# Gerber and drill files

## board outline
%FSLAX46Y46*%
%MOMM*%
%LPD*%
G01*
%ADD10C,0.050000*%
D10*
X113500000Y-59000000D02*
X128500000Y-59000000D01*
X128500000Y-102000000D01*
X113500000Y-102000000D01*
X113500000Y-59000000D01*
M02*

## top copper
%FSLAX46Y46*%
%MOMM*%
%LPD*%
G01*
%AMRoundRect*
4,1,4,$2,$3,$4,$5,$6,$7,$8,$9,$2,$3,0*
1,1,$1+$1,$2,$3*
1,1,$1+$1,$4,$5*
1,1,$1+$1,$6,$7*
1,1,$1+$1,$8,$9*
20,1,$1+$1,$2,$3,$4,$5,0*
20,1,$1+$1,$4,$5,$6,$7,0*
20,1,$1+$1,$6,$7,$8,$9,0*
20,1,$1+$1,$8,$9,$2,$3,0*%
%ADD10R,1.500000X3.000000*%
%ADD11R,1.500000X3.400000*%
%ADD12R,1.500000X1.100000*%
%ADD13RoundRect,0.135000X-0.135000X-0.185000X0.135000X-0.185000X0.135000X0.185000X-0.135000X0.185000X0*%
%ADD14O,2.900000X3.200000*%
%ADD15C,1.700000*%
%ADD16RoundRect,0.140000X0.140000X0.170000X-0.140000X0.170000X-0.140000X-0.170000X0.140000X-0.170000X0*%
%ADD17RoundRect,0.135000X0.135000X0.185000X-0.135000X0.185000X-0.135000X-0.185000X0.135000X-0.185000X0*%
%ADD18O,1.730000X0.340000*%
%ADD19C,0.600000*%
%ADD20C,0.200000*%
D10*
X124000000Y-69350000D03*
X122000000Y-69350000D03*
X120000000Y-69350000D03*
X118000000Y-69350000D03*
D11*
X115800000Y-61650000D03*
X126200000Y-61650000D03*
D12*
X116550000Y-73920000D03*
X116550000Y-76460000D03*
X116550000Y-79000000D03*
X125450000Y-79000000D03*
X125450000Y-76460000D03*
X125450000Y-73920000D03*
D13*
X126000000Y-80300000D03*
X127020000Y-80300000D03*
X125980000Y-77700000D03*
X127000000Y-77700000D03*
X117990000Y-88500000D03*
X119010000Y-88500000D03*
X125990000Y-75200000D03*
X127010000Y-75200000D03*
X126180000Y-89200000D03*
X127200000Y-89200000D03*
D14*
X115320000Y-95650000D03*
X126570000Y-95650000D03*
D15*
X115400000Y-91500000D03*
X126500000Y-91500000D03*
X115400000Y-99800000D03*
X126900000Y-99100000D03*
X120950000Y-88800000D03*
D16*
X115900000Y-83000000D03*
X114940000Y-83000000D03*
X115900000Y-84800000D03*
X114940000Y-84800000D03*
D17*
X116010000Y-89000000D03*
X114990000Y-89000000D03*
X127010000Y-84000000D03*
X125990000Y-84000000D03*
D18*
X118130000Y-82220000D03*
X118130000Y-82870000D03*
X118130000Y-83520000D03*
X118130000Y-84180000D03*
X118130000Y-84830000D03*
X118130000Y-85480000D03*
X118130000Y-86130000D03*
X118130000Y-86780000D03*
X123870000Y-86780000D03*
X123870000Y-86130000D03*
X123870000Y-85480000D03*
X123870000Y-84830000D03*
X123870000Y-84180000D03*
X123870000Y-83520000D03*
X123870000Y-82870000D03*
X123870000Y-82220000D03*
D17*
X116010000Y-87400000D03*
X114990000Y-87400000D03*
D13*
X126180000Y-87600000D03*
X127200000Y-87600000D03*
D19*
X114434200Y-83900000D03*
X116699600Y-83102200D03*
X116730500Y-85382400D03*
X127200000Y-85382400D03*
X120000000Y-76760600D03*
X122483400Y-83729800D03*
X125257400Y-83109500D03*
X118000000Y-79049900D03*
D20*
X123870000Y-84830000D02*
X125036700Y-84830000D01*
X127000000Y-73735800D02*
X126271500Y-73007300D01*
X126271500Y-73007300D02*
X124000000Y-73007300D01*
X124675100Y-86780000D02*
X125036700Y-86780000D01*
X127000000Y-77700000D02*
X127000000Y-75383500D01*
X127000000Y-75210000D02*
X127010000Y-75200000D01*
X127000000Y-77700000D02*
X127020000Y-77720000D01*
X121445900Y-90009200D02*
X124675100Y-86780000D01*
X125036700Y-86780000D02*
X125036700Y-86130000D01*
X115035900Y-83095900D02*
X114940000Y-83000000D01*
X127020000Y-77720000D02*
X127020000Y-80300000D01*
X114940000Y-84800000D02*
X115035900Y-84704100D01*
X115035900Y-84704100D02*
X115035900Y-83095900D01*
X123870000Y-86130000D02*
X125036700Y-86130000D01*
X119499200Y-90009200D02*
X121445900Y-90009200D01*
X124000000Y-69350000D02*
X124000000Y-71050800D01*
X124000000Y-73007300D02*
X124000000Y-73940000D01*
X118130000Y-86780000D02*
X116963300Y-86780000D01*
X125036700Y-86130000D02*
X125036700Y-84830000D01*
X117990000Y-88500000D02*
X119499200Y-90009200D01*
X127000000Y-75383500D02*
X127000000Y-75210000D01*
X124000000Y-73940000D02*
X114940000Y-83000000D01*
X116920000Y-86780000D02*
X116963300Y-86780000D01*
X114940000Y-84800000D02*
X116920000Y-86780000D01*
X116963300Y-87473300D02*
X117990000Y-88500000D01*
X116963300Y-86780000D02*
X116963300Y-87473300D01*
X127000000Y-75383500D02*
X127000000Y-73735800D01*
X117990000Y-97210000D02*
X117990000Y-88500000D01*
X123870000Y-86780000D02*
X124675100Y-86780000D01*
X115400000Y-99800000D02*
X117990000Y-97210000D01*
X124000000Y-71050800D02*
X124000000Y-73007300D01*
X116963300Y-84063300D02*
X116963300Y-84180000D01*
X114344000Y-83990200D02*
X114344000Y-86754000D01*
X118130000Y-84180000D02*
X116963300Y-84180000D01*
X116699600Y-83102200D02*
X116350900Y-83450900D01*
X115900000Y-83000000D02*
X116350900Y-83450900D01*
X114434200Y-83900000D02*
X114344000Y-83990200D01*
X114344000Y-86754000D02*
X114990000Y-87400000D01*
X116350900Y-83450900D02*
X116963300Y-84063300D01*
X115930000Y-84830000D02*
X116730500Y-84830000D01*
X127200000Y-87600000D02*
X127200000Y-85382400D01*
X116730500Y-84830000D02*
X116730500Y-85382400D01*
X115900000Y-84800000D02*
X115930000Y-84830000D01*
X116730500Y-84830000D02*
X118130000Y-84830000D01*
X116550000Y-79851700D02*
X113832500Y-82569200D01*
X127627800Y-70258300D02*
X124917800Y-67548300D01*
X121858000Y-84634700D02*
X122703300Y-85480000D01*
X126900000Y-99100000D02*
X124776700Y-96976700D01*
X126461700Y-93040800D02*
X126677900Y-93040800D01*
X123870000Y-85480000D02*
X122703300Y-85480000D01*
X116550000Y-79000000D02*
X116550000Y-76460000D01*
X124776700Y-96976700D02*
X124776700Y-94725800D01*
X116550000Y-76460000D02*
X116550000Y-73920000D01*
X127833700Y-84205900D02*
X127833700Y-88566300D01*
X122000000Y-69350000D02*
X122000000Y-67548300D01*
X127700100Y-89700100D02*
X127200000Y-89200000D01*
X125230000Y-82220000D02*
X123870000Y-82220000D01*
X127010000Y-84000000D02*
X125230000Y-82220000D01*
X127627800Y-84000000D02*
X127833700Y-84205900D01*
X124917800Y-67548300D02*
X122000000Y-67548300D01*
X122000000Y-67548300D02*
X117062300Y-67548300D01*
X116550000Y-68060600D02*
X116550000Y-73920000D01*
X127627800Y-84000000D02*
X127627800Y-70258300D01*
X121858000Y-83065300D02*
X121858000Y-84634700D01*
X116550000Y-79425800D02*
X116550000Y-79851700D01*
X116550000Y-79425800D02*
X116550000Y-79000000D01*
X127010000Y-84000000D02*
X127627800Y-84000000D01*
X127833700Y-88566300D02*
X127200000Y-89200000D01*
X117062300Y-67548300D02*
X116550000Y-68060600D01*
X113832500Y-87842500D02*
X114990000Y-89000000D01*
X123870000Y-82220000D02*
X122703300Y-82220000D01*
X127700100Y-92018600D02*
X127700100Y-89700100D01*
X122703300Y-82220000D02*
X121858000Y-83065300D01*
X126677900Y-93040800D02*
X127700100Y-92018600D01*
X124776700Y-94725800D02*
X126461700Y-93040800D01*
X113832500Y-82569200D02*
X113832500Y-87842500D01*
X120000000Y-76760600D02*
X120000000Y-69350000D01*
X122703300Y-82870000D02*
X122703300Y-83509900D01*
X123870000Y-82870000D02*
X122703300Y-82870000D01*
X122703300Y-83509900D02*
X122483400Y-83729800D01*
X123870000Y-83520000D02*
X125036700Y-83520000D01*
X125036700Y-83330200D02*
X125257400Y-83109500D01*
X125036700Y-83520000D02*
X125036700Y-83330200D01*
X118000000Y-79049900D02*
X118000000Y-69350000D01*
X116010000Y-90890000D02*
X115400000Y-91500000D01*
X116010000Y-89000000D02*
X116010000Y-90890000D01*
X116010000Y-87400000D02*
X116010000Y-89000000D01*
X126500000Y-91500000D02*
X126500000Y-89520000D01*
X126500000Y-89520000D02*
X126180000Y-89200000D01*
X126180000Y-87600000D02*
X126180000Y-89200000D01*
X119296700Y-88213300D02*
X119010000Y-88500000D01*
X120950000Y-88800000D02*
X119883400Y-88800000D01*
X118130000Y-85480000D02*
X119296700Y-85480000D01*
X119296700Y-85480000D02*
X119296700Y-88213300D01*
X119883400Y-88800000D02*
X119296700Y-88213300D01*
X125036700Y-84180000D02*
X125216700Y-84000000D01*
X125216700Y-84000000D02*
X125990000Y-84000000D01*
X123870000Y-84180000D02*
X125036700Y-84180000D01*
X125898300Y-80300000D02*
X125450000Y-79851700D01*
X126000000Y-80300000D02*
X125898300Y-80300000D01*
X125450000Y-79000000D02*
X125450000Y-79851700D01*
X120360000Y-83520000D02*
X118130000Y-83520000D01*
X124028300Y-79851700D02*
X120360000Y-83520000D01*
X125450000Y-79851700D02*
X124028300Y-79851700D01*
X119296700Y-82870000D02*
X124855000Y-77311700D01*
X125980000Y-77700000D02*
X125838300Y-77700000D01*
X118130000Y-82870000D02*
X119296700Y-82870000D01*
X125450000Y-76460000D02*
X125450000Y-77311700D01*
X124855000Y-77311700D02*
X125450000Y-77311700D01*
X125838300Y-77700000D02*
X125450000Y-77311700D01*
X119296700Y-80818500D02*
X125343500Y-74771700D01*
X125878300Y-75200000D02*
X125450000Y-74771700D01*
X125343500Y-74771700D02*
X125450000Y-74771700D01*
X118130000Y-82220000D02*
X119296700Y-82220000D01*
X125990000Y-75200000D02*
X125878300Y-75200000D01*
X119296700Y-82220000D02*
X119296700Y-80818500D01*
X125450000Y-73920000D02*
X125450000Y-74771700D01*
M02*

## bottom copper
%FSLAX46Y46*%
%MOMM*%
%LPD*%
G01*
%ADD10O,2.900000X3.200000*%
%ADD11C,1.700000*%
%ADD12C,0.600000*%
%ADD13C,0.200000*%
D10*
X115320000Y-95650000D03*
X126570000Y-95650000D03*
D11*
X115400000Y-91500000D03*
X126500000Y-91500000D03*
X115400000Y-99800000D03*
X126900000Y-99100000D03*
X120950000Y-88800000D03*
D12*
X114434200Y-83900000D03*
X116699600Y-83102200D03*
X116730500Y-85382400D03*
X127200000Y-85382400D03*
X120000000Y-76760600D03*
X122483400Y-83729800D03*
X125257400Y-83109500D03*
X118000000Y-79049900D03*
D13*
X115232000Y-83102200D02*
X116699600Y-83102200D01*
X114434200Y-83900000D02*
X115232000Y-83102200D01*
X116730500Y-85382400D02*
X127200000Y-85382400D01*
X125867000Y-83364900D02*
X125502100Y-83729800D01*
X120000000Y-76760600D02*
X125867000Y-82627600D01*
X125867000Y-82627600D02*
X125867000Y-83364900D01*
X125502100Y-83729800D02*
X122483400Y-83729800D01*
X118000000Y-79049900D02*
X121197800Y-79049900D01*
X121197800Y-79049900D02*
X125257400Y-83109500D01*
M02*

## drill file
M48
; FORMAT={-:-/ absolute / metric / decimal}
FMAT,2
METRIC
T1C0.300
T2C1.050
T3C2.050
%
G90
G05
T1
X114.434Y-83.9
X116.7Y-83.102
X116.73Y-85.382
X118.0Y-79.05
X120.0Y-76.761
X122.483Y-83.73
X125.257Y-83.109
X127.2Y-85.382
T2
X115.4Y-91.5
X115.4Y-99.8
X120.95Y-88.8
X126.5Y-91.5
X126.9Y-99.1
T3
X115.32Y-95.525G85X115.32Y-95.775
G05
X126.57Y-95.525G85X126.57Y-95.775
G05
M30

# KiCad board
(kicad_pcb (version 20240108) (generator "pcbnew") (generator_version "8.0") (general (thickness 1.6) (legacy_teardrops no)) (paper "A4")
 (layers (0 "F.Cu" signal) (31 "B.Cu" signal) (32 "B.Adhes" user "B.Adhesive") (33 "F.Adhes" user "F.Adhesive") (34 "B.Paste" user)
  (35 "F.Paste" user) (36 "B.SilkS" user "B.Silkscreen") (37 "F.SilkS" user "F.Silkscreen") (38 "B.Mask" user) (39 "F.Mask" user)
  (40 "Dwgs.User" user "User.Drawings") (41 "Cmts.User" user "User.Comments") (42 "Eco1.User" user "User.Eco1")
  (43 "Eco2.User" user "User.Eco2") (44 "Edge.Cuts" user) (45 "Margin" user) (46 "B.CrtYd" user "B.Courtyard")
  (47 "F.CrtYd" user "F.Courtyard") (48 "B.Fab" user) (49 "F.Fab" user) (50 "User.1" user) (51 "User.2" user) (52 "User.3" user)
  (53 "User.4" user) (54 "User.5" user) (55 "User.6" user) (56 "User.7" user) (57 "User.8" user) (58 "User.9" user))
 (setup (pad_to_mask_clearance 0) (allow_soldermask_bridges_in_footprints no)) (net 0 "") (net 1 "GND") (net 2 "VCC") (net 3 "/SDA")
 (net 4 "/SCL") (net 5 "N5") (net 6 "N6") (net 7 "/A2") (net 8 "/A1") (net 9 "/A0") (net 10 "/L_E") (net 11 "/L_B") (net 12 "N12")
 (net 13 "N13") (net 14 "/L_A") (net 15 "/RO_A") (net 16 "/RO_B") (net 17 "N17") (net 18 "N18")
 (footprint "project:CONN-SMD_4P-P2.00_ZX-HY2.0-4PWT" (layer "F.Cu") (at 121 65.5 180)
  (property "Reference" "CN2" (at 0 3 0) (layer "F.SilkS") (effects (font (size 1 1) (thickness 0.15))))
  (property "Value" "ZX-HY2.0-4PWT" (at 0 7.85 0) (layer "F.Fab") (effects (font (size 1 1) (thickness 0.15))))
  (pad "1" smd rect (at -3 -3.85 180) (size 1.5 3) (layers "F.Cu" "F.Paste" "F.Mask") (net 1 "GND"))
  (pad "2" smd rect (at -1 -3.85 180) (size 1.5 3) (layers "F.Cu" "F.Paste" "F.Mask") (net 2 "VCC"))
  (pad "3" smd rect (at 1 -3.85 180) (size 1.5 3) (layers "F.Cu" "F.Paste" "F.Mask") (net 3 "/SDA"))
  (pad "4" smd rect (at 3 -3.85 180) (size 1.5 3) (layers "F.Cu" "F.Paste" "F.Mask") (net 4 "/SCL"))
  (pad "5" smd rect (at 5.2 3.85 180) (size 1.5 3.4) (layers "F.Cu" "F.Paste" "F.Mask") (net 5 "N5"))
  (pad "6" smd rect (at -5.2 3.85 180) (size 1.5 3.4) (layers "F.Cu" "F.Paste" "F.Mask") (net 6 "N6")))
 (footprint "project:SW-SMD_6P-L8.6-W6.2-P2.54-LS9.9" (layer "F.Cu") (at 121 76.46 -90)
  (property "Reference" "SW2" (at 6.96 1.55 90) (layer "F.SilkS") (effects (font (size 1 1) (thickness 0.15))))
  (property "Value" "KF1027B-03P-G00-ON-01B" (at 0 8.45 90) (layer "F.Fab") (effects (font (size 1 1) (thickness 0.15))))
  (pad "1" smd rect (at -2.54 4.45 180) (size 1.5 1.1) (layers "F.Cu" "F.Paste" "F.Mask") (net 2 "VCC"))
  (pad "2" smd rect (at 0 4.45 180) (size 1.5 1.1) (layers "F.Cu" "F.Paste" "F.Mask") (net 2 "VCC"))
  (pad "3" smd rect (at 2.54 4.45 180) (size 1.5 1.1) (layers "F.Cu" "F.Paste" "F.Mask") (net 2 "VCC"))
  (pad "4" smd rect (at 2.54 -4.45 180) (size 1.5 1.1) (layers "F.Cu" "F.Paste" "F.Mask") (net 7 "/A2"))
  (pad "5" smd rect (at 0 -4.45 180) (size 1.5 1.1) (layers "F.Cu" "F.Paste" "F.Mask") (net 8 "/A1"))
  (pad "6" smd rect (at -2.54 -4.45 180) (size 1.5 1.1) (layers "F.Cu" "F.Paste" "F.Mask") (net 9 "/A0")))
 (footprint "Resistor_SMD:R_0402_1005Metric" (layer "F.Cu") (at 126.51 80.3)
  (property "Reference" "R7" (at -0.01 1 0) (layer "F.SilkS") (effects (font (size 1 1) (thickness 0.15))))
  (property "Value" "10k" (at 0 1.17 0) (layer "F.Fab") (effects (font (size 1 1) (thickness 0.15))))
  (pad "1" smd roundrect (at -0.51 0) (size 0.54 0.64) (layers "F.Cu" "F.Paste" "F.Mask") (roundrect_rratio 0.25) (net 7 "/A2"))
  (pad "2" smd roundrect (at 0.51 0) (size 0.54 0.64) (layers "F.Cu" "F.Paste" "F.Mask") (roundrect_rratio 0.25) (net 1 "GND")))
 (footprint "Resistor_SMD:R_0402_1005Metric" (layer "F.Cu") (at 126.49 77.7)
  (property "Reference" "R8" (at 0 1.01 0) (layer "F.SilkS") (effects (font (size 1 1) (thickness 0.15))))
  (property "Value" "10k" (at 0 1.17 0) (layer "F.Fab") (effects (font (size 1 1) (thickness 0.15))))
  (pad "1" smd roundrect (at -0.51 0) (size 0.54 0.64) (layers "F.Cu" "F.Paste" "F.Mask") (roundrect_rratio 0.25) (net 8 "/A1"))
  (pad "2" smd roundrect (at 0.51 0) (size 0.54 0.64) (layers "F.Cu" "F.Paste" "F.Mask") (roundrect_rratio 0.25) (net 1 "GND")))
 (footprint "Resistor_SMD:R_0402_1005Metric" (layer "F.Cu") (at 118.5 88.5)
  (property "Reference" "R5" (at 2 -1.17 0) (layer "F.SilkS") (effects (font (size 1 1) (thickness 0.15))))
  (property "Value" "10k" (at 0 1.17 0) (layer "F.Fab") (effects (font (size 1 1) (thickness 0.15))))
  (pad "1" smd roundrect (at -0.51 0) (size 0.54 0.64) (layers "F.Cu" "F.Paste" "F.Mask") (roundrect_rratio 0.25) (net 1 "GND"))
  (pad "2" smd roundrect (at 0.51 0) (size 0.54 0.64) (layers "F.Cu" "F.Paste" "F.Mask") (roundrect_rratio 0.25) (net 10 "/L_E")))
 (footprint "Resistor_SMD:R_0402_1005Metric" (layer "F.Cu") (at 126.5 75.2)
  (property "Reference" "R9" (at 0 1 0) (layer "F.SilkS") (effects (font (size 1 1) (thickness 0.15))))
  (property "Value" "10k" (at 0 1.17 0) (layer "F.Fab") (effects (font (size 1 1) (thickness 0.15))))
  (pad "1" smd roundrect (at -0.51 0) (size 0.54 0.64) (layers "F.Cu" "F.Paste" "F.Mask") (roundrect_rratio 0.25) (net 9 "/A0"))
  (pad "2" smd roundrect (at 0.51 0) (size 0.54 0.64) (layers "F.Cu" "F.Paste" "F.Mask") (roundrect_rratio 0.25) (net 1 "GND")))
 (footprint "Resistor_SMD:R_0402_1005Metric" (layer "F.Cu") (at 126.69 89.2)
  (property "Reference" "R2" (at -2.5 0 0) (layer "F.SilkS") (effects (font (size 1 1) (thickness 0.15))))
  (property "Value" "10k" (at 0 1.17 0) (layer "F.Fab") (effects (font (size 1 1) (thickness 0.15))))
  (pad "1" smd roundrect (at -0.51 0) (size 0.54 0.64) (layers "F.Cu" "F.Paste" "F.Mask") (roundrect_rratio 0.25) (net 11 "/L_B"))
  (pad "2" smd roundrect (at 0.51 0) (size 0.54 0.64) (layers "F.Cu" "F.Paste" "F.Mask") (roundrect_rratio 0.25) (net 2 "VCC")))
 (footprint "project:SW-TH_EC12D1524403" (layer "F.Cu") (at 121.11 94.3)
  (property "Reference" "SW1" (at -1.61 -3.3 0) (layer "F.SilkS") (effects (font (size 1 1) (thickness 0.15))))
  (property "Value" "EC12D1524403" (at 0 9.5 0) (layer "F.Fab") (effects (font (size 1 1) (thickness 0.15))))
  (pad "6" thru_hole oval (at -5.79 1.35) (size 2.9 3.2) (drill oval 2.049983 2.299995) (layers "*.Cu" "*.Mask") (remove_unused_layers no)
   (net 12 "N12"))
  (pad "7" thru_hole oval (at 5.46 1.35) (size 2.9 3.2) (drill oval 2.049983 2.299995) (layers "*.Cu" "*.Mask") (remove_unused_layers no)
   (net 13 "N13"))
  (pad "A" thru_hole circle (at -5.71 -2.8) (size 1.7 1.7) (drill 1.049985) (layers "*.Cu" "*.Mask") (remove_unused_layers no)
   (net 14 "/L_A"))
  (pad "B" thru_hole circle (at 5.39 -2.8) (size 1.7 1.7) (drill 1.049985) (layers "*.Cu" "*.Mask") (remove_unused_layers no)
   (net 11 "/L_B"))
  (pad "C" thru_hole circle (at -5.71 5.5) (size 1.7 1.7) (drill 1.049985) (layers "*.Cu" "*.Mask") (remove_unused_layers no) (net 1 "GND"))
  (pad "D" thru_hole circle (at 5.79 4.8) (size 1.7 1.7) (drill 1.049985) (layers "*.Cu" "*.Mask") (remove_unused_layers no) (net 2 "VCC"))
  (pad "E" thru_hole circle (at -0.16 -5.5) (size 1.7 1.7) (drill 1.049985) (layers "*.Cu" "*.Mask") (remove_unused_layers no)
   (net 10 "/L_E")))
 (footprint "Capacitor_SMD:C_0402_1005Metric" (layer "F.Cu") (at 115.42 83 180)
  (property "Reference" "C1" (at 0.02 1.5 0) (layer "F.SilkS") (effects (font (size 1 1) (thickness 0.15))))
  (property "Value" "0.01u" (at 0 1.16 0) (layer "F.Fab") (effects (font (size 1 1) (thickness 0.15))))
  (pad "1" smd roundrect (at -0.48 0 180) (size 0.56 0.62) (layers "F.Cu" "F.Paste" "F.Mask") (roundrect_rratio 0.25) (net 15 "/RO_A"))
  (pad "2" smd roundrect (at 0.48 0 180) (size 0.56 0.62) (layers "F.Cu" "F.Paste" "F.Mask") (roundrect_rratio 0.25) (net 1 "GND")))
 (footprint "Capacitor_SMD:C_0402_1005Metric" (layer "F.Cu") (at 115.42 84.8 180)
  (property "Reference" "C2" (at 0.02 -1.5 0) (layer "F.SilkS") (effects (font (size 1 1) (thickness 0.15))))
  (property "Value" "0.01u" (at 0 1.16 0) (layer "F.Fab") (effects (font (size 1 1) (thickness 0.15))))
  (pad "1" smd roundrect (at -0.48 0 180) (size 0.56 0.62) (layers "F.Cu" "F.Paste" "F.Mask") (roundrect_rratio 0.25) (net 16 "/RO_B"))
  (pad "2" smd roundrect (at 0.48 0 180) (size 0.56 0.62) (layers "F.Cu" "F.Paste" "F.Mask") (roundrect_rratio 0.25) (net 1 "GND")))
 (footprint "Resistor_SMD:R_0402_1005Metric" (layer "F.Cu") (at 115.5 89 180)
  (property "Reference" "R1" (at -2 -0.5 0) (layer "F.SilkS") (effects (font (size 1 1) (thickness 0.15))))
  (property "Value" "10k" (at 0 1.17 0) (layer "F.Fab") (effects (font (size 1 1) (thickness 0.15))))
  (pad "1" smd roundrect (at -0.51 0 180) (size 0.54 0.64) (layers "F.Cu" "F.Paste" "F.Mask") (roundrect_rratio 0.25) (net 14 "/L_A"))
  (pad "2" smd roundrect (at 0.51 0 180) (size 0.54 0.64) (layers "F.Cu" "F.Paste" "F.Mask") (roundrect_rratio 0.25) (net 2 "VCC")))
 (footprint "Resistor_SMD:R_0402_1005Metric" (layer "F.Cu") (at 126.5 84 180)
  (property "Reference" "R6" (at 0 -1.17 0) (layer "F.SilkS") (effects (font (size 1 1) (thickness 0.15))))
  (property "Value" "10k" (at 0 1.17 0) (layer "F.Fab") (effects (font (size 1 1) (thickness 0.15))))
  (pad "1" smd roundrect (at -0.51 0 180) (size 0.54 0.64) (layers "F.Cu" "F.Paste" "F.Mask") (roundrect_rratio 0.25) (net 2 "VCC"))
  (pad "2" smd roundrect (at 0.51 0 180) (size 0.54 0.64) (layers "F.Cu" "F.Paste" "F.Mask") (roundrect_rratio 0.25) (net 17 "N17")))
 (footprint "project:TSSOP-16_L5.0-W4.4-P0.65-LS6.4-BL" (layer "F.Cu") (at 121 84.5 -90)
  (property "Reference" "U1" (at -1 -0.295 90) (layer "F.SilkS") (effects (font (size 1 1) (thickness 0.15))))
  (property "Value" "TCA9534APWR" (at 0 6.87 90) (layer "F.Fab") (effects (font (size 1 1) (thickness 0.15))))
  (pad "1" smd oval (at -2.28 2.87 270) (size 0.34 1.73) (layers "F.Cu" "F.Paste" "F.Mask") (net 9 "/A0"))
  (pad "2" smd oval (at -1.63 2.87 270) (size 0.34 1.73) (layers "F.Cu" "F.Paste" "F.Mask") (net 8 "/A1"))
  (pad "3" smd oval (at -0.98 2.87 270) (size 0.34 1.73) (layers "F.Cu" "F.Paste" "F.Mask") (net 7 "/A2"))
  (pad "4" smd oval (at -0.32 2.87 270) (size 0.34 1.73) (layers "F.Cu" "F.Paste" "F.Mask") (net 15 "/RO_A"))
  (pad "5" smd oval (at 0.33 2.87 270) (size 0.34 1.73) (layers "F.Cu" "F.Paste" "F.Mask") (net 16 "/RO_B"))
  (pad "6" smd oval (at 0.98 2.87 270) (size 0.34 1.73) (layers "F.Cu" "F.Paste" "F.Mask") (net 10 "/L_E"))
  (pad "7" smd oval (at 1.63 2.87 270) (size 0.34 1.73) (layers "F.Cu" "F.Paste" "F.Mask") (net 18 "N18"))
  (pad "8" smd oval (at 2.28 2.87 270) (size 0.34 1.73) (layers "F.Cu" "F.Paste" "F.Mask") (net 1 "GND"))
  (pad "9" smd oval (at 2.28 -2.87 270) (size 0.34 1.73) (layers "F.Cu" "F.Paste" "F.Mask") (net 1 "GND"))
  (pad "10" smd oval (at 1.63 -2.87 270) (size 0.34 1.73) (layers "F.Cu" "F.Paste" "F.Mask") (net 1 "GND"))
  (pad "11" smd oval (at 0.98 -2.87 270) (size 0.34 1.73) (layers "F.Cu" "F.Paste" "F.Mask") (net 2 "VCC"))
  (pad "12" smd oval (at 0.33 -2.87 270) (size 0.34 1.73) (layers "F.Cu" "F.Paste" "F.Mask") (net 1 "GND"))
  (pad "13" smd oval (at -0.32 -2.87 270) (size 0.34 1.73) (layers "F.Cu" "F.Paste" "F.Mask") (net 17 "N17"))
  (pad "14" smd oval (at -0.98 -2.87 270) (size 0.34 1.73) (layers "F.Cu" "F.Paste" "F.Mask") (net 4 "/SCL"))
  (pad "15" smd oval (at -1.63 -2.87 270) (size 0.34 1.73) (layers "F.Cu" "F.Paste" "F.Mask") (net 3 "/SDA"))
  (pad "16" smd oval (at -2.28 -2.87 270) (size 0.34 1.73) (layers "F.Cu" "F.Paste" "F.Mask") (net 2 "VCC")))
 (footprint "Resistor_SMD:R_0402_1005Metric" (layer "F.Cu") (at 115.5 87.4 180)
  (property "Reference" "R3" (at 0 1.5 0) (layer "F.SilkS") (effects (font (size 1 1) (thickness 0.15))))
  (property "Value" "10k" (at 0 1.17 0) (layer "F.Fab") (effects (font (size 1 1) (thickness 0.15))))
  (pad "1" smd roundrect (at -0.51 0 180) (size 0.54 0.64) (layers "F.Cu" "F.Paste" "F.Mask") (roundrect_rratio 0.25) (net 14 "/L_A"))
  (pad "2" smd roundrect (at 0.51 0 180) (size 0.54 0.64) (layers "F.Cu" "F.Paste" "F.Mask") (roundrect_rratio 0.25) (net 15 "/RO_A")))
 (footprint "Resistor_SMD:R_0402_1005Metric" (layer "F.Cu") (at 126.69 87.6)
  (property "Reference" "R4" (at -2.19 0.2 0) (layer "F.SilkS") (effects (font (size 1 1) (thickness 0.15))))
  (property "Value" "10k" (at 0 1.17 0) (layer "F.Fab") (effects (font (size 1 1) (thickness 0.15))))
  (pad "1" smd roundrect (at -0.51 0) (size 0.54 0.64) (layers "F.Cu" "F.Paste" "F.Mask") (roundrect_rratio 0.25) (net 11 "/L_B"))
  (pad "2" smd roundrect (at 0.51 0) (size 0.54 0.64) (layers "F.Cu" "F.Paste" "F.Mask") (roundrect_rratio 0.25) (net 16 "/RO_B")))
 (gr_rect (start 113.5 59) (end 128.5 102) (stroke (width 0.05) (type default)) (fill none) (layer "Edge.Cuts"))
 (segment (start 123.87 84.83) (end 125.0367 84.83) (width 0.2) (layer "F.Cu") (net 1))
 (segment (start 127 73.7358) (end 126.2715 73.0073) (width 0.2) (layer "F.Cu") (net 1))
 (segment (start 126.2715 73.0073) (end 124 73.0073) (width 0.2) (layer "F.Cu") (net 1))
 (segment (start 124.6751 86.78) (end 125.0367 86.78) (width 0.2) (layer "F.Cu") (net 1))
 (segment (start 127 77.7) (end 127 75.3835) (width 0.2) (layer "F.Cu") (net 1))
 (segment (start 127 75.21) (end 127.01 75.2) (width 0.2) (layer "F.Cu") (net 1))
 (segment (start 127 77.7) (end 127.02 77.72) (width 0.2) (layer "F.Cu") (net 1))
 (segment (start 121.4459 90.0092) (end 124.6751 86.78) (width 0.2) (layer "F.Cu") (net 1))
 (segment (start 125.0367 86.78) (end 125.0367 86.13) (width 0.2) (layer "F.Cu") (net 1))
 (segment (start 115.0359 83.0959) (end 114.94 83) (width 0.2) (layer "F.Cu") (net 1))
 (segment (start 127.02 77.72) (end 127.02 80.3) (width 0.2) (layer "F.Cu") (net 1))
 (segment (start 114.94 84.8) (end 115.0359 84.7041) (width 0.2) (layer "F.Cu") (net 1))
 (segment (start 115.0359 84.7041) (end 115.0359 83.0959) (width 0.2) (layer "F.Cu") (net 1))
 (segment (start 123.87 86.13) (end 125.0367 86.13) (width 0.2) (layer "F.Cu") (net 1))
 (segment (start 119.4992 90.0092) (end 121.4459 90.0092) (width 0.2) (layer "F.Cu") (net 1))
 (segment (start 124 69.35) (end 124 71.0508) (width 0.2) (layer "F.Cu") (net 1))
 (segment (start 124 73.0073) (end 124 73.94) (width 0.2) (layer "F.Cu") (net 1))
 (segment (start 118.13 86.78) (end 116.9633 86.78) (width 0.2) (layer "F.Cu") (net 1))
 (segment (start 125.0367 86.13) (end 125.0367 84.83) (width 0.2) (layer "F.Cu") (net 1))
 (segment (start 117.99 88.5) (end 119.4992 90.0092) (width 0.2) (layer "F.Cu") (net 1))
 (segment (start 127 75.3835) (end 127 75.21) (width 0.2) (layer "F.Cu") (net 1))
 (segment (start 124 73.94) (end 114.94 83) (width 0.2) (layer "F.Cu") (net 1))
 (segment (start 116.92 86.78) (end 116.9633 86.78) (width 0.2) (layer "F.Cu") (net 1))
 (segment (start 114.94 84.8) (end 116.92 86.78) (width 0.2) (layer "F.Cu") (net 1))
 (segment (start 116.9633 87.4733) (end 117.99 88.5) (width 0.2) (layer "F.Cu") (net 1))
 (segment (start 116.9633 86.78) (end 116.9633 87.4733) (width 0.2) (layer "F.Cu") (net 1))
 (segment (start 127 75.3835) (end 127 73.7358) (width 0.2) (layer "F.Cu") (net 1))
 (segment (start 117.99 97.21) (end 117.99 88.5) (width 0.2) (layer "F.Cu") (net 1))
 (segment (start 123.87 86.78) (end 124.6751 86.78) (width 0.2) (layer "F.Cu") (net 1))
 (segment (start 115.4 99.8) (end 117.99 97.21) (width 0.2) (layer "F.Cu") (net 1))
 (segment (start 124 71.0508) (end 124 73.0073) (width 0.2) (layer "F.Cu") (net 1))
 (segment (start 116.9633 84.0633) (end 116.9633 84.18) (width 0.2) (layer "F.Cu") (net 15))
 (segment (start 114.344 83.9902) (end 114.344 86.754) (width 0.2) (layer "F.Cu") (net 15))
 (segment (start 118.13 84.18) (end 116.9633 84.18) (width 0.2) (layer "F.Cu") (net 15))
 (segment (start 116.6996 83.1022) (end 116.3509 83.4509) (width 0.2) (layer "F.Cu") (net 15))
 (segment (start 115.9 83) (end 116.3509 83.4509) (width 0.2) (layer "F.Cu") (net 15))
 (segment (start 114.4342 83.9) (end 114.344 83.9902) (width 0.2) (layer "F.Cu") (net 15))
 (segment (start 114.344 86.754) (end 114.99 87.4) (width 0.2) (layer "F.Cu") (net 15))
 (segment (start 116.3509 83.4509) (end 116.9633 84.0633) (width 0.2) (layer "F.Cu") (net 15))
 (via (at 114.4342 83.9) (size 0.6) (drill 0.3) (layers "F.Cu" "B.Cu") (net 15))
 (via (at 116.6996 83.1022) (size 0.6) (drill 0.3) (layers "F.Cu" "B.Cu") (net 15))
 (segment (start 115.232 83.1022) (end 116.6996 83.1022) (width 0.2) (layer "B.Cu") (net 15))
 (segment (start 114.4342 83.9) (end 115.232 83.1022) (width 0.2) (layer "B.Cu") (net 15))
 (segment (start 115.93 84.83) (end 116.7305 84.83) (width 0.2) (layer "F.Cu") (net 16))
 (segment (start 127.2 87.6) (end 127.2 85.3824) (width 0.2) (layer "F.Cu") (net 16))
 (segment (start 116.7305 84.83) (end 116.7305 85.3824) (width 0.2) (layer "F.Cu") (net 16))
 (segment (start 115.9 84.8) (end 115.93 84.83) (width 0.2) (layer "F.Cu") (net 16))
 (segment (start 116.7305 84.83) (end 118.13 84.83) (width 0.2) (layer "F.Cu") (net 16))
 (via (at 116.7305 85.3824) (size 0.6) (drill 0.3) (layers "F.Cu" "B.Cu") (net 16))
 (via (at 127.2 85.3824) (size 0.6) (drill 0.3) (layers "F.Cu" "B.Cu") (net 16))
 (segment (start 116.7305 85.3824) (end 127.2 85.3824) (width 0.2) (layer "B.Cu") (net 16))
 (segment (start 116.55 79.8517) (end 113.8325 82.5692) (width 0.2) (layer "F.Cu") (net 2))
 (segment (start 127.6278 70.2583) (end 124.9178 67.5483) (width 0.2) (layer "F.Cu") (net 2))
 (segment (start 121.858 84.6347) (end 122.7033 85.48) (width 0.2) (layer "F.Cu") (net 2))
 (segment (start 126.9 99.1) (end 124.7767 96.9767) (width 0.2) (layer "F.Cu") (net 2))
 (segment (start 126.4617 93.0408) (end 126.6779 93.0408) (width 0.2) (layer "F.Cu") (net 2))
 (segment (start 123.87 85.48) (end 122.7033 85.48) (width 0.2) (layer "F.Cu") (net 2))
 (segment (start 116.55 79) (end 116.55 76.46) (width 0.2) (layer "F.Cu") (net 2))
 (segment (start 124.7767 96.9767) (end 124.7767 94.7258) (width 0.2) (layer "F.Cu") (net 2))
 (segment (start 116.55 76.46) (end 116.55 73.92) (width 0.2) (layer "F.Cu") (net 2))
 (segment (start 127.8337 84.2059) (end 127.8337 88.5663) (width 0.2) (layer "F.Cu") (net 2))
 (segment (start 122 69.35) (end 122 67.5483) (width 0.2) (layer "F.Cu") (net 2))
 (segment (start 127.7001 89.7001) (end 127.2 89.2) (width 0.2) (layer "F.Cu") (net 2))
 (segment (start 125.23 82.22) (end 123.87 82.22) (width 0.2) (layer "F.Cu") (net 2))
 (segment (start 127.01 84) (end 125.23 82.22) (width 0.2) (layer "F.Cu") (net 2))
 (segment (start 127.6278 84) (end 127.8337 84.2059) (width 0.2) (layer "F.Cu") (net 2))
 (segment (start 124.9178 67.5483) (end 122 67.5483) (width 0.2) (layer "F.Cu") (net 2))
 (segment (start 122 67.5483) (end 117.0623 67.5483) (width 0.2) (layer "F.Cu") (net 2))
 (segment (start 116.55 68.0606) (end 116.55 73.92) (width 0.2) (layer "F.Cu") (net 2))
 (segment (start 127.6278 84) (end 127.6278 70.2583) (width 0.2) (layer "F.Cu") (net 2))
 (segment (start 121.858 83.0653) (end 121.858 84.6347) (width 0.2) (layer "F.Cu") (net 2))
 (segment (start 116.55 79.4258) (end 116.55 79.8517) (width 0.2) (layer "F.Cu") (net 2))
 (segment (start 116.55 79.4258) (end 116.55 79) (width 0.2) (layer "F.Cu") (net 2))
 (segment (start 127.01 84) (end 127.6278 84) (width 0.2) (layer "F.Cu") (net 2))
 (segment (start 127.8337 88.5663) (end 127.2 89.2) (width 0.2) (layer "F.Cu") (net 2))
 (segment (start 117.0623 67.5483) (end 116.55 68.0606) (width 0.2) (layer "F.Cu") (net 2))
 (segment (start 113.8325 87.8425) (end 114.99 89) (width 0.2) (layer "F.Cu") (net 2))
 (segment (start 123.87 82.22) (end 122.7033 82.22) (width 0.2) (layer "F.Cu") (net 2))
 (segment (start 127.7001 92.0186) (end 127.7001 89.7001) (width 0.2) (layer "F.Cu") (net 2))
 (segment (start 122.7033 82.22) (end 121.858 83.0653) (width 0.2) (layer "F.Cu") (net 2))
 (segment (start 126.6779 93.0408) (end 127.7001 92.0186) (width 0.2) (layer "F.Cu") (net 2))
 (segment (start 124.7767 94.7258) (end 126.4617 93.0408) (width 0.2) (layer "F.Cu") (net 2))
 (segment (start 113.8325 82.5692) (end 113.8325 87.8425) (width 0.2) (layer "F.Cu") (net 2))
 (segment (start 120 76.7606) (end 120 69.35) (width 0.2) (layer "F.Cu") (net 3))
 (segment (start 122.7033 82.87) (end 122.7033 83.5099) (width 0.2) (layer "F.Cu") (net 3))
 (segment (start 123.87 82.87) (end 122.7033 82.87) (width 0.2) (layer "F.Cu") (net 3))
 (segment (start 122.7033 83.5099) (end 122.4834 83.7298) (width 0.2) (layer "F.Cu") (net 3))
 (via (at 120 76.7606) (size 0.6) (drill 0.3) (layers "F.Cu" "B.Cu") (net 3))
 (via (at 122.4834 83.7298) (size 0.6) (drill 0.3) (layers "F.Cu" "B.Cu") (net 3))
 (segment (start 125.867 83.3649) (end 125.5021 83.7298) (width 0.2) (layer "B.Cu") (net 3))
 (segment (start 120 76.7606) (end 125.867 82.6276) (width 0.2) (layer "B.Cu") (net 3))
 (segment (start 125.867 82.6276) (end 125.867 83.3649) (width 0.2) (layer "B.Cu") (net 3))
 (segment (start 125.5021 83.7298) (end 122.4834 83.7298) (width 0.2) (layer "B.Cu") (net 3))
 (segment (start 123.87 83.52) (end 125.0367 83.52) (width 0.2) (layer "F.Cu") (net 4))
 (segment (start 125.0367 83.3302) (end 125.2574 83.1095) (width 0.2) (layer "F.Cu") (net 4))
 (segment (start 125.0367 83.52) (end 125.0367 83.3302) (width 0.2) (layer "F.Cu") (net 4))
 (segment (start 118 79.0499) (end 118 69.35) (width 0.2) (layer "F.Cu") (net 4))
 (via (at 125.2574 83.1095) (size 0.6) (drill 0.3) (layers "F.Cu" "B.Cu") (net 4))
 (via (at 118 79.0499) (size 0.6) (drill 0.3) (layers "F.Cu" "B.Cu") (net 4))
 (segment (start 118 79.0499) (end 121.1978 79.0499) (width 0.2) (layer "B.Cu") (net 4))
 (segment (start 121.1978 79.0499) (end 125.2574 83.1095) (width 0.2) (layer "B.Cu") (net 4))
 (segment (start 116.01 90.89) (end 115.4 91.5) (width 0.2) (layer "F.Cu") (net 14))
 (segment (start 116.01 89) (end 116.01 90.89) (width 0.2) (layer "F.Cu") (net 14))
 (segment (start 116.01 87.4) (end 116.01 89) (width 0.2) (layer "F.Cu") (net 14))
 (segment (start 126.5 91.5) (end 126.5 89.52) (width 0.2) (layer "F.Cu") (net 11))
 (segment (start 126.5 89.52) (end 126.18 89.2) (width 0.2) (layer "F.Cu") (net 11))
 (segment (start 126.18 87.6) (end 126.18 89.2) (width 0.2) (layer "F.Cu") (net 11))
 (segment (start 119.2967 88.2133) (end 119.01 88.5) (width 0.2) (layer "F.Cu") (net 10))
 (segment (start 120.95 88.8) (end 119.8834 88.8) (width 0.2) (layer "F.Cu") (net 10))
 (segment (start 118.13 85.48) (end 119.2967 85.48) (width 0.2) (layer "F.Cu") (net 10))
 (segment (start 119.2967 85.48) (end 119.2967 88.2133) (width 0.2) (layer "F.Cu") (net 10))
 (segment (start 119.8834 88.8) (end 119.2967 88.2133) (width 0.2) (layer "F.Cu") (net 10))
 (segment (start 125.0367 84.18) (end 125.2167 84) (width 0.2) (layer "F.Cu") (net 17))
 (segment (start 125.2167 84) (end 125.99 84) (width 0.2) (layer "F.Cu") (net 17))
 (segment (start 123.87 84.18) (end 125.0367 84.18) (width 0.2) (layer "F.Cu") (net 17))
 (segment (start 125.8983 80.3) (end 125.45 79.8517) (width 0.2) (layer "F.Cu") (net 7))
 (segment (start 126 80.3) (end 125.8983 80.3) (width 0.2) (layer "F.Cu") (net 7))
 (segment (start 125.45 79) (end 125.45 79.8517) (width 0.2) (layer "F.Cu") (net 7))
 (segment (start 120.36 83.52) (end 118.13 83.52) (width 0.2) (layer "F.Cu") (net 7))
 (segment (start 124.0283 79.8517) (end 120.36 83.52) (width 0.2) (layer "F.Cu") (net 7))
 (segment (start 125.45 79.8517) (end 124.0283 79.8517) (width 0.2) (layer "F.Cu") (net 7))
 (segment (start 119.2967 82.87) (end 124.855 77.3117) (width 0.2) (layer "F.Cu") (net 8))
 (segment (start 125.98 77.7) (end 125.8383 77.7) (width 0.2) (layer "F.Cu") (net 8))
 (segment (start 118.13 82.87) (end 119.2967 82.87) (width 0.2) (layer "F.Cu") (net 8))
 (segment (start 125.45 76.46) (end 125.45 77.3117) (width 0.2) (layer "F.Cu") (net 8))
 (segment (start 124.855 77.3117) (end 125.45 77.3117) (width 0.2) (layer "F.Cu") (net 8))
 (segment (start 125.8383 77.7) (end 125.45 77.3117) (width 0.2) (layer "F.Cu") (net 8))
 (segment (start 119.2967 80.8185) (end 125.3435 74.7717) (width 0.2) (layer "F.Cu") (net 9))
 (segment (start 125.8783 75.2) (end 125.45 74.7717) (width 0.2) (layer "F.Cu") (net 9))
 (segment (start 125.3435 74.7717) (end 125.45 74.7717) (width 0.2) (layer "F.Cu") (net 9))
 (segment (start 118.13 82.22) (end 119.2967 82.22) (width 0.2) (layer "F.Cu") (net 9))
 (segment (start 125.99 75.2) (end 125.8783 75.2) (width 0.2) (layer "F.Cu") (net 9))
 (segment (start 119.2967 82.22) (end 119.2967 80.8185) (width 0.2) (layer "F.Cu") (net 9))
 (segment (start 125.45 73.92) (end 125.45 74.7717) (width 0.2) (layer "F.Cu") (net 9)))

